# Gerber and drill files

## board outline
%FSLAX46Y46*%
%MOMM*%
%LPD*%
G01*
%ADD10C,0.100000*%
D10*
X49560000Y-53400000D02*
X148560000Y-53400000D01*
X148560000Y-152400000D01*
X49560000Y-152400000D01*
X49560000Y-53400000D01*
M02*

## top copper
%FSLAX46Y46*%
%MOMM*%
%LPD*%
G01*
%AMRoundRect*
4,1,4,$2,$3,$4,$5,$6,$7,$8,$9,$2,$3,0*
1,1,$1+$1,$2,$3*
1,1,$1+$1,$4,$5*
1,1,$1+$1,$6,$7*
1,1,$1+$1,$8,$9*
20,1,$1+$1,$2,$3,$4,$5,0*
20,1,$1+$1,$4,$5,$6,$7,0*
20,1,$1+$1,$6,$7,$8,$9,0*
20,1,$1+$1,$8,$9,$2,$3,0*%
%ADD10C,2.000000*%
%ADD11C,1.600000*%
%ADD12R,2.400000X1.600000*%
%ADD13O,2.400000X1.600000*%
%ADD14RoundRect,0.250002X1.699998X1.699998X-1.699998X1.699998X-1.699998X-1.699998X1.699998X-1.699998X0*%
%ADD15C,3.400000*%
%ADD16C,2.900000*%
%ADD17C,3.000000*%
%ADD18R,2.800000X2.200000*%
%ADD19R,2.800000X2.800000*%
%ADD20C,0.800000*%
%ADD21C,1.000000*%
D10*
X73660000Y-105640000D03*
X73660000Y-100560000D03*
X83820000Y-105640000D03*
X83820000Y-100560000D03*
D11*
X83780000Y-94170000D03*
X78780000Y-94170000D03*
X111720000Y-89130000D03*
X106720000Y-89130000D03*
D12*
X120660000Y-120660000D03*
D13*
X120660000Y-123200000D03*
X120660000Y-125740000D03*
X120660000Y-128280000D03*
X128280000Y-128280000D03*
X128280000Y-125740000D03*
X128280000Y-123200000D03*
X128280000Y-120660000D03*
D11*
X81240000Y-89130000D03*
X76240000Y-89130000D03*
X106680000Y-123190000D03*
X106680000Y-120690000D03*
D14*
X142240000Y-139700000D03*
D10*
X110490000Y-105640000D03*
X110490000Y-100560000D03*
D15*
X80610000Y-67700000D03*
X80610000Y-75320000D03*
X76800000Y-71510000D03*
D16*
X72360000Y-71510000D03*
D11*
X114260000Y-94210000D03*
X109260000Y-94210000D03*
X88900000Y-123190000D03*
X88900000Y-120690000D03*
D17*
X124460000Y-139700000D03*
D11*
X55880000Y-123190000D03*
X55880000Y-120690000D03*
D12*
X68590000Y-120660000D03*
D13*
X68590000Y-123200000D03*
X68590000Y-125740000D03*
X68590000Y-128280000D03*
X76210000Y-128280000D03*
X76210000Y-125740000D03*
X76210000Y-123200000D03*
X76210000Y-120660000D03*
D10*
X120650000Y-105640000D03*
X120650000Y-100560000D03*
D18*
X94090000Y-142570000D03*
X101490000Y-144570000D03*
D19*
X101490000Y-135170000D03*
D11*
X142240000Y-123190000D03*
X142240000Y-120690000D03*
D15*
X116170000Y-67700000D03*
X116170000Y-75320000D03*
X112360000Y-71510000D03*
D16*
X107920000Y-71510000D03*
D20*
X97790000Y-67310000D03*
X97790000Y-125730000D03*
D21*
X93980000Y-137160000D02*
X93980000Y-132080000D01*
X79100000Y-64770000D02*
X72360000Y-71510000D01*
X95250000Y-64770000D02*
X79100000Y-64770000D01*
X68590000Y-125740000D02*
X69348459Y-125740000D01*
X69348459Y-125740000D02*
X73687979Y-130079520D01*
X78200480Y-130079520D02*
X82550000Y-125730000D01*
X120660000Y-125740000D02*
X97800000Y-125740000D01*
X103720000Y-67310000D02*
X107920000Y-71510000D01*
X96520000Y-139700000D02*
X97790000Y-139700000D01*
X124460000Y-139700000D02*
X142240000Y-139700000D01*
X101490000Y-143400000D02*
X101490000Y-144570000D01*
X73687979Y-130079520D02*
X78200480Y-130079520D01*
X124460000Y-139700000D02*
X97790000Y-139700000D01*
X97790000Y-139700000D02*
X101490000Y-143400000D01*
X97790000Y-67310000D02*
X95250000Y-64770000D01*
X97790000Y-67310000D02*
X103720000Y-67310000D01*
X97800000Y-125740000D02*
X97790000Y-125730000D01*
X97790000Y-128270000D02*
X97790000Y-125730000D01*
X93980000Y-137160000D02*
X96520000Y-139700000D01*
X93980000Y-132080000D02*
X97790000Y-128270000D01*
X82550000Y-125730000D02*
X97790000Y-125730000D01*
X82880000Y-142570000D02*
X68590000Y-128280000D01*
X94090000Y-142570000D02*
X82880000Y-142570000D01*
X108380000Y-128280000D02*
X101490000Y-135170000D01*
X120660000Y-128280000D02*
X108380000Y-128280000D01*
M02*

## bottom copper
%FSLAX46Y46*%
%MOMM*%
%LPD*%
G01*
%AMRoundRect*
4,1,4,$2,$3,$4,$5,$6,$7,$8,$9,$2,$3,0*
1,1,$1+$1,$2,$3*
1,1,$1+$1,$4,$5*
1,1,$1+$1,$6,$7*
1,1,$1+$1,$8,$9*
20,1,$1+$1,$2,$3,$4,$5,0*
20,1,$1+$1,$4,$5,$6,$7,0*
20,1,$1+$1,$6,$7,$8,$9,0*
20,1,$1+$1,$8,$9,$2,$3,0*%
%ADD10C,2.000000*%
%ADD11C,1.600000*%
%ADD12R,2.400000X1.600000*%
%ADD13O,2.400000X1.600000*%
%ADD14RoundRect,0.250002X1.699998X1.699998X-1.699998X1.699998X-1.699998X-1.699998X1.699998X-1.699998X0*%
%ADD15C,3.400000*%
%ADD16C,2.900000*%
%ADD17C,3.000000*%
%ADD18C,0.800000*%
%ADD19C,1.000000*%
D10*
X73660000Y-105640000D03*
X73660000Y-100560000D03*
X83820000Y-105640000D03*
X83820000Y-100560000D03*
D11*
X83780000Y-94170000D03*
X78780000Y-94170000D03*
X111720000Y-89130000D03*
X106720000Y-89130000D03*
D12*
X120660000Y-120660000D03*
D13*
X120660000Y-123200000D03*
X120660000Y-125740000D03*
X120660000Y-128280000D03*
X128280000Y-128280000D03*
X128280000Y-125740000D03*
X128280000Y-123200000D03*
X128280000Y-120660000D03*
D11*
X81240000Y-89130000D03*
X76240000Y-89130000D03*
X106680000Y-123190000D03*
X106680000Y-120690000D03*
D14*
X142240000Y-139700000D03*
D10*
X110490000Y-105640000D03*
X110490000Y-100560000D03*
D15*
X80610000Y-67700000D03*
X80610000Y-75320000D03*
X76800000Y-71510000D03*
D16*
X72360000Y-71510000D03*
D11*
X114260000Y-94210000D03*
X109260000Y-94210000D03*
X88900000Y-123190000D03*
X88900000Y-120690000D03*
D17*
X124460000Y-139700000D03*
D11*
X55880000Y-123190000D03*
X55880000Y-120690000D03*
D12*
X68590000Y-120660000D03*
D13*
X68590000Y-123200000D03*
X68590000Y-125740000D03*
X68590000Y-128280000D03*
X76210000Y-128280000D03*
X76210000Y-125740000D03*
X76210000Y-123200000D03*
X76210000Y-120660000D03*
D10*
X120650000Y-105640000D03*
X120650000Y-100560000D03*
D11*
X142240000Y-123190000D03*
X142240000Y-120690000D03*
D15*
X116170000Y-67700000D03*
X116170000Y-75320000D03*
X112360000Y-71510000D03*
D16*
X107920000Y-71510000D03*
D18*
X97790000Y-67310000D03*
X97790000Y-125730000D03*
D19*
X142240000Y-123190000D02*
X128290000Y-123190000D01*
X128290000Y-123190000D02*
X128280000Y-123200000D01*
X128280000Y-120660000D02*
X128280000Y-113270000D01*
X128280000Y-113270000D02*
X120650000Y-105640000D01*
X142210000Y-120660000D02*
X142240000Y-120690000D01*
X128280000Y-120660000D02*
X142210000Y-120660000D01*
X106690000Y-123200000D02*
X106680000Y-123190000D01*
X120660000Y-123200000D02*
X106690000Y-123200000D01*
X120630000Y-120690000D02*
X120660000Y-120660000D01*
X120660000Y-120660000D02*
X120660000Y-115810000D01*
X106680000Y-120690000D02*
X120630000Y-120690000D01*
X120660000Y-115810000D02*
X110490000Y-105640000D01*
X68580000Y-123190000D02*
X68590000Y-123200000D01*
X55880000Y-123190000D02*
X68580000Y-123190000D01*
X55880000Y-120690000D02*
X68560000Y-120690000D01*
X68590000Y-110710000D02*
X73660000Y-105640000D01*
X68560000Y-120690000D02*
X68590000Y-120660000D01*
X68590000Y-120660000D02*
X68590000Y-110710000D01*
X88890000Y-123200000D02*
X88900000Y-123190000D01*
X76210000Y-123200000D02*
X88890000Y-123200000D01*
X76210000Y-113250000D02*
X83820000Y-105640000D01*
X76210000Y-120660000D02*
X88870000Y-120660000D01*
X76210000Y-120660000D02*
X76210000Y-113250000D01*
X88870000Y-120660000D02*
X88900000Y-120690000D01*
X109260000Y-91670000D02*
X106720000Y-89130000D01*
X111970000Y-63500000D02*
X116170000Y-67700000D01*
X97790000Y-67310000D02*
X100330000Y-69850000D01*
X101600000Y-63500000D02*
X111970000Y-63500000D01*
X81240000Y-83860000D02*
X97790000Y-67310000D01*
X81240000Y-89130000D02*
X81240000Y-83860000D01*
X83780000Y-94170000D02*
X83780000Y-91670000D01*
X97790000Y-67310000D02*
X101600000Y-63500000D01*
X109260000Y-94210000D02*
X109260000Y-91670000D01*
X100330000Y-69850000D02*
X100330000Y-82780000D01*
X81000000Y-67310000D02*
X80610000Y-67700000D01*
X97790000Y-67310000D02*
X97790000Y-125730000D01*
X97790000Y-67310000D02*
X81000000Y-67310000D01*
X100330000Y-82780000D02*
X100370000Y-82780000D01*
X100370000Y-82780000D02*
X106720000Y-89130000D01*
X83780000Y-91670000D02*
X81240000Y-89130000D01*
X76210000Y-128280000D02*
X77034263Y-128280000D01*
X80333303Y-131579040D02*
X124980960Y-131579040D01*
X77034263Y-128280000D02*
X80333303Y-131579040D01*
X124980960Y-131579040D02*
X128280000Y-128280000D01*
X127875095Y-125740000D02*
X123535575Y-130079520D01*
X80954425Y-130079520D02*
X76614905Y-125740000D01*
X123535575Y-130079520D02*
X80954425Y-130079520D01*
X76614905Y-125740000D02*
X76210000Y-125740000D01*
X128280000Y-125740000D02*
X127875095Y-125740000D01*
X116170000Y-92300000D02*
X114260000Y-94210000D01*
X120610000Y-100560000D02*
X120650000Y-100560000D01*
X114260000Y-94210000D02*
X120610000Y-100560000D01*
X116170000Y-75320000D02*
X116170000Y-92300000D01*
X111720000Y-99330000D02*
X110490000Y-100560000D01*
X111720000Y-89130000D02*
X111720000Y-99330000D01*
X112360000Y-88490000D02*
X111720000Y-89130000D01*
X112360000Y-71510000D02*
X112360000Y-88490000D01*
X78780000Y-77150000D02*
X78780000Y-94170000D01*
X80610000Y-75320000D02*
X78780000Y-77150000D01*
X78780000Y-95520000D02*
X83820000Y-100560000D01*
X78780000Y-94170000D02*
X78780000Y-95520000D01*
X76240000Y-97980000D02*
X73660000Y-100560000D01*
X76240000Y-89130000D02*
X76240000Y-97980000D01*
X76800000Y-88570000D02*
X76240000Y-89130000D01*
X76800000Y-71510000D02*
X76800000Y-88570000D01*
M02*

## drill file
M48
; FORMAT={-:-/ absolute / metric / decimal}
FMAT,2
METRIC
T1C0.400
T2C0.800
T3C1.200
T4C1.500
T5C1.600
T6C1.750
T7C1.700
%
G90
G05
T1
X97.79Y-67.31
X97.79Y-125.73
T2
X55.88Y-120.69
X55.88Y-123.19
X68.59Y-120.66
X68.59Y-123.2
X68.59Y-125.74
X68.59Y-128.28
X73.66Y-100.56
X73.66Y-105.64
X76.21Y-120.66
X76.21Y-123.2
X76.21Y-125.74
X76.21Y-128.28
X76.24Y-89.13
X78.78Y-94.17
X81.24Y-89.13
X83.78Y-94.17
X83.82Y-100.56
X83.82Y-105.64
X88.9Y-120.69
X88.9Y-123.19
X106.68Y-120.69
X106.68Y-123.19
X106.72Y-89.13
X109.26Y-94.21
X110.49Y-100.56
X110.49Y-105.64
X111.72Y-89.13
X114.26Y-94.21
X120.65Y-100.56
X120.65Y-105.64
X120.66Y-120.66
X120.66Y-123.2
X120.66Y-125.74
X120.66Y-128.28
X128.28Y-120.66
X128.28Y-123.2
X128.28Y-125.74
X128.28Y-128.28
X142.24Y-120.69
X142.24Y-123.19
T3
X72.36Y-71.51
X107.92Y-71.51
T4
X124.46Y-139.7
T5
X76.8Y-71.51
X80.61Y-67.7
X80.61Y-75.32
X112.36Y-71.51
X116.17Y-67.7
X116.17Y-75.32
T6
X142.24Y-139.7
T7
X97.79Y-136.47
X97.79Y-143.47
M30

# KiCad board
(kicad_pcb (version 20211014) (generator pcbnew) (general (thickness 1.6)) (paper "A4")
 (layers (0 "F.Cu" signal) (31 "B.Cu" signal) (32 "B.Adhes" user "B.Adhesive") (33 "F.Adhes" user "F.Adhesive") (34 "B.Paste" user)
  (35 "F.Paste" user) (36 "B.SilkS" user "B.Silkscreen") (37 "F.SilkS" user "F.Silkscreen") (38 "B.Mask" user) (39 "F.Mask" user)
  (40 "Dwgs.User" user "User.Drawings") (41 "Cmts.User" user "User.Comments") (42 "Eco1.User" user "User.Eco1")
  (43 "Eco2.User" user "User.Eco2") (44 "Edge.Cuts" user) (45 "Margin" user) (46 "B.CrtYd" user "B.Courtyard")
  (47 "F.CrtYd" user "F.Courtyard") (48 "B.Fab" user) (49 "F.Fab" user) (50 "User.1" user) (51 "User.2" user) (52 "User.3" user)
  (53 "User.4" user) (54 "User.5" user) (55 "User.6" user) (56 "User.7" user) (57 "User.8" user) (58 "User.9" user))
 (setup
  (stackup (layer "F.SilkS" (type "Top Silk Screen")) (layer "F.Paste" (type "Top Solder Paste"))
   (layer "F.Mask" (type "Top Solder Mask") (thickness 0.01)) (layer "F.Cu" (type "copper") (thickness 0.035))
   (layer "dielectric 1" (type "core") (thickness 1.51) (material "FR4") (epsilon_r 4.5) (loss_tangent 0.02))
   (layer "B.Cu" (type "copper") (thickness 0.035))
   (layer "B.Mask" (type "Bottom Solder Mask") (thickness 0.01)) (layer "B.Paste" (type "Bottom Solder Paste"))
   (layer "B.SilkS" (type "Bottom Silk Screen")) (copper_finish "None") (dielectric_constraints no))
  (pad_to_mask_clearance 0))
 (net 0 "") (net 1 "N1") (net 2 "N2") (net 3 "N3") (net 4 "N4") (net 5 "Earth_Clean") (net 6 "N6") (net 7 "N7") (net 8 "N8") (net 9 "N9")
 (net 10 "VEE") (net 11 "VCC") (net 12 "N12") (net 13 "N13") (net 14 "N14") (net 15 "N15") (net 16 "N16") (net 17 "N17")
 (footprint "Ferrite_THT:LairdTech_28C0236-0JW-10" (layer "F.Cu") (at 73.66 105.64 90)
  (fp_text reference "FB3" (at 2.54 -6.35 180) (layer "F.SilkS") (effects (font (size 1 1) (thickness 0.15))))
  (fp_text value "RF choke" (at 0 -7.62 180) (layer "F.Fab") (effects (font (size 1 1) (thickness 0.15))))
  (pad "1" thru_hole circle (at 0 0 90) (size 2 2) (drill 0.8) (layers *.Cu *.Mask) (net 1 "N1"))
  (pad "2" thru_hole circle (at 5.08 0 90) (size 2 2) (drill 0.8) (layers *.Cu *.Mask) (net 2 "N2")))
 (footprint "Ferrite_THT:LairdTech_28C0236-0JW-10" (layer "F.Cu") (at 83.82 105.64 90)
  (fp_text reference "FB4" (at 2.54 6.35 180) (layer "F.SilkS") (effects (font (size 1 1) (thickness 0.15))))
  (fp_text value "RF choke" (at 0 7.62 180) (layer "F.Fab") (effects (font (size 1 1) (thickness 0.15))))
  (pad "1" thru_hole circle (at 0 0 90) (size 2 2) (drill 0.8) (layers *.Cu *.Mask) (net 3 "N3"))
  (pad "2" thru_hole circle (at 5.08 0 90) (size 2 2) (drill 0.8) (layers *.Cu *.Mask) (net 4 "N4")))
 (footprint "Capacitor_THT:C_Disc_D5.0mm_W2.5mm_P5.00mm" (layer "F.Cu") (at 83.78 94.17 180)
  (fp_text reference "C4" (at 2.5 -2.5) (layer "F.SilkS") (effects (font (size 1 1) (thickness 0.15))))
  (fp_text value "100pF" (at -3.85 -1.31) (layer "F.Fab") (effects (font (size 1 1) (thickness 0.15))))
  (pad "1" thru_hole circle (at 0 0 180) (size 1.6 1.6) (drill 0.8) (layers *.Cu *.Mask) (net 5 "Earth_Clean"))
  (pad "2" thru_hole circle (at 5 0 180) (size 1.6 1.6) (drill 0.8) (layers *.Cu *.Mask) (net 4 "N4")))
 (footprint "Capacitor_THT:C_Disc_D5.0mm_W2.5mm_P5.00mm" (layer "F.Cu") (at 111.72 89.13 180)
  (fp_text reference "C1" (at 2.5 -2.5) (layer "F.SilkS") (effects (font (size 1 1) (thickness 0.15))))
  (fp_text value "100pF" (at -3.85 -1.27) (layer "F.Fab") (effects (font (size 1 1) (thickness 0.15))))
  (pad "1" thru_hole circle (at 0 0 180) (size 1.6 1.6) (drill 0.8) (layers *.Cu *.Mask) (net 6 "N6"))
  (pad "2" thru_hole circle (at 5 0 180) (size 1.6 1.6) (drill 0.8) (layers *.Cu *.Mask) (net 5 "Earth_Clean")))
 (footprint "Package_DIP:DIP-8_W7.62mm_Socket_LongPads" (layer "F.Cu") (at 120.66 120.66)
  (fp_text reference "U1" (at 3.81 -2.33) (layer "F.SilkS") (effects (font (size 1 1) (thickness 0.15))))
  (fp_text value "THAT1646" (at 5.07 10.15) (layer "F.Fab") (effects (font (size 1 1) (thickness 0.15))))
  (pad "1" thru_hole rect (at 0 0) (size 2.4 1.6) (drill 0.8) (layers *.Cu *.Mask) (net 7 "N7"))
  (pad "2" thru_hole oval (at 0 2.54) (size 2.4 1.6) (drill 0.8) (layers *.Cu *.Mask) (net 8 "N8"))
  (pad "3" thru_hole oval (at 0 5.08) (size 2.4 1.6) (drill 0.8) (layers *.Cu *.Mask) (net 5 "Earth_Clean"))
  (pad "4" thru_hole oval (at 0 7.62) (size 2.4 1.6) (drill 0.8) (layers *.Cu *.Mask) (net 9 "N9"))
  (pad "5" thru_hole oval (at 7.62 7.62) (size 2.4 1.6) (drill 0.8) (layers *.Cu *.Mask) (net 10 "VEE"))
  (pad "6" thru_hole oval (at 7.62 5.08) (size 2.4 1.6) (drill 0.8) (layers *.Cu *.Mask) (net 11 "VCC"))
  (pad "7" thru_hole oval (at 7.62 2.54) (size 2.4 1.6) (drill 0.8) (layers *.Cu *.Mask) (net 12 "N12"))
  (pad "8" thru_hole oval (at 7.62 0) (size 2.4 1.6) (drill 0.8) (layers *.Cu *.Mask) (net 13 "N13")))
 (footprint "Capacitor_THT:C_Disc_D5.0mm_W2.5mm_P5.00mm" (layer "F.Cu") (at 81.24 89.13 180)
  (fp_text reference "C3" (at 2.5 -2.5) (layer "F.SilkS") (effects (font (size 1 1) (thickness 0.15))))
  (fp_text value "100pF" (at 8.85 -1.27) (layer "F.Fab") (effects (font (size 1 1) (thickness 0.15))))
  (pad "1" thru_hole circle (at 0 0 180) (size 1.6 1.6) (drill 0.8) (layers *.Cu *.Mask) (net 5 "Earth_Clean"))
  (pad "2" thru_hole circle (at 5 0 180) (size 1.6 1.6) (drill 0.8) (layers *.Cu *.Mask) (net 2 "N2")))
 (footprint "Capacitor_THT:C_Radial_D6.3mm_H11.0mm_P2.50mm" (layer "F.Cu") (at 106.68 123.19 90)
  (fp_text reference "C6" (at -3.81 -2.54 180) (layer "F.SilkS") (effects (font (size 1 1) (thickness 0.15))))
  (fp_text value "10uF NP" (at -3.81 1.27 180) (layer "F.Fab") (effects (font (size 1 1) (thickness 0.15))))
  (pad "1" thru_hole circle (at 0 0 90) (size 1.6 1.6) (drill 0.8) (layers *.Cu *.Mask) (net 8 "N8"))
  (pad "2" thru_hole circle (at 2.5 0 90) (size 1.6 1.6) (drill 0.8) (layers *.Cu *.Mask) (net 7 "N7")))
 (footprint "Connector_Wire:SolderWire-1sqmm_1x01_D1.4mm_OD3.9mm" (layer "F.Cu") (at 142.24 139.7 180)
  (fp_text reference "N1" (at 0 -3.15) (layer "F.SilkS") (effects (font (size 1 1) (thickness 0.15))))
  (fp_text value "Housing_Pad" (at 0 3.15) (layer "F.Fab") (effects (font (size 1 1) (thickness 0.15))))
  (pad "1" thru_hole roundrect (at 0 0 180) (size 3.9 3.9) (drill 1.75) (layers *.Cu *.Mask) (roundrect_rratio 0.06410307692)
   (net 5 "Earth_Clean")))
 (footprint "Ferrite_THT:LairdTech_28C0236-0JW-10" (layer "F.Cu") (at 110.49 105.64 90)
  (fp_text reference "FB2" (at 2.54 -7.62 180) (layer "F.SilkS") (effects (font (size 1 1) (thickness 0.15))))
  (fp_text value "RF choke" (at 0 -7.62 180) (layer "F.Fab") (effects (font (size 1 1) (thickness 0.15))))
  (pad "1" thru_hole circle (at 0 0 90) (size 2 2) (drill 0.8) (layers *.Cu *.Mask) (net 7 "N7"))
  (pad "2" thru_hole circle (at 5.08 0 90) (size 2 2) (drill 0.8) (layers *.Cu *.Mask) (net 6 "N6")))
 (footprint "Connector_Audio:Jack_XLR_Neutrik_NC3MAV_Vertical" (layer "F.Cu") (at 80.61 67.7 -90)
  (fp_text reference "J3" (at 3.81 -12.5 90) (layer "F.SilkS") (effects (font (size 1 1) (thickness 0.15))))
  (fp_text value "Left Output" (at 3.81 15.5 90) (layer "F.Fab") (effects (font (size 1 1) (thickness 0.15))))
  (pad "1" thru_hole circle (at 0 0 270) (size 3.4 3.4) (drill 1.6) (layers *.Cu *.Mask) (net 5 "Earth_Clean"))
  (pad "2" thru_hole circle (at 7.62 0 270) (size 3.4 3.4) (drill 1.6) (layers *.Cu *.Mask) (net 4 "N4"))
  (pad "3" thru_hole circle (at 3.81 3.81 270) (size 3.4 3.4) (drill 1.6) (layers *.Cu *.Mask) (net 2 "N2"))
  (pad "G" thru_hole circle (at 3.81 8.25 270) (size 2.9 2.9) (drill 1.2) (layers *.Cu *.Mask) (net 5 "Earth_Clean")))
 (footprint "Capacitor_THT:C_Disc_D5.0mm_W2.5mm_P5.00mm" (layer "F.Cu") (at 114.26 94.21 180)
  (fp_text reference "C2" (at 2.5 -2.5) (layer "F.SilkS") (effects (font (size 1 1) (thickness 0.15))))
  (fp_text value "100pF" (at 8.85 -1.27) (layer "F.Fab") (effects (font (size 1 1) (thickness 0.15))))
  (pad "1" thru_hole circle (at 0 0 180) (size 1.6 1.6) (drill 0.8) (layers *.Cu *.Mask) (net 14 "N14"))
  (pad "2" thru_hole circle (at 5 0 180) (size 1.6 1.6) (drill 0.8) (layers *.Cu *.Mask) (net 5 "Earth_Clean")))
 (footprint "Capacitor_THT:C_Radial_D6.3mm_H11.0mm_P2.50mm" (layer "F.Cu") (at 88.9 123.19 90)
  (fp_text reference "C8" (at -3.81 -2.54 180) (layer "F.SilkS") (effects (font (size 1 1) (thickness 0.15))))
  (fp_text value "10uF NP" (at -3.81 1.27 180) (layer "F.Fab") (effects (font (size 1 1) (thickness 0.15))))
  (pad "1" thru_hole circle (at 0 0 90) (size 1.6 1.6) (drill 0.8) (layers *.Cu *.Mask) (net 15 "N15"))
  (pad "2" thru_hole circle (at 2.5 0 90) (size 1.6 1.6) (drill 0.8) (layers *.Cu *.Mask) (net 3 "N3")))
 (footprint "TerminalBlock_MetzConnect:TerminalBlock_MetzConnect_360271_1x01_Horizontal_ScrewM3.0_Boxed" (layer "F.Cu")
  (at 124.46 139.7 180)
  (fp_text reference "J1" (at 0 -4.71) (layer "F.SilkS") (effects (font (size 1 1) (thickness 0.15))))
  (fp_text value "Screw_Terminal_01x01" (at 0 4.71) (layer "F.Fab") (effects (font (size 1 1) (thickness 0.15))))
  (pad "1" thru_hole circle (at 0 0 180) (size 3 3) (drill 1.5) (layers *.Cu *.Mask) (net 5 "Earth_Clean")))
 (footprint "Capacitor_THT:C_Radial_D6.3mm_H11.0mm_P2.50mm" (layer "F.Cu") (at 55.88 123.19 90)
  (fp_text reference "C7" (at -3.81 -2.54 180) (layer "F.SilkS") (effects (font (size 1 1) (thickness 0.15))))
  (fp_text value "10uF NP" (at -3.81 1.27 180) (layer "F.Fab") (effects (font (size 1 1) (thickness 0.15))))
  (pad "1" thru_hole circle (at 0 0 90) (size 1.6 1.6) (drill 0.8) (layers *.Cu *.Mask) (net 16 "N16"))
  (pad "2" thru_hole circle (at 2.5 0 90) (size 1.6 1.6) (drill 0.8) (layers *.Cu *.Mask) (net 1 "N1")))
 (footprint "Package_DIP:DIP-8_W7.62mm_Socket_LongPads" (layer "F.Cu") (at 68.59 120.66)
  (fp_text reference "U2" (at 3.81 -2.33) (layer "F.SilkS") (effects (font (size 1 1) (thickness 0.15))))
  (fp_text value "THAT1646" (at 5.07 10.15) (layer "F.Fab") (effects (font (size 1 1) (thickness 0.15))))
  (pad "1" thru_hole rect (at 0 0) (size 2.4 1.6) (drill 0.8) (layers *.Cu *.Mask) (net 1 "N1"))
  (pad "2" thru_hole oval (at 0 2.54) (size 2.4 1.6) (drill 0.8) (layers *.Cu *.Mask) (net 16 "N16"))
  (pad "3" thru_hole oval (at 0 5.08) (size 2.4 1.6) (drill 0.8) (layers *.Cu *.Mask) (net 5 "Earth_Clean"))
  (pad "4" thru_hole oval (at 0 7.62) (size 2.4 1.6) (drill 0.8) (layers *.Cu *.Mask) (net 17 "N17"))
  (pad "5" thru_hole oval (at 7.62 7.62) (size 2.4 1.6) (drill 0.8) (layers *.Cu *.Mask) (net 10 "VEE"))
  (pad "6" thru_hole oval (at 7.62 5.08) (size 2.4 1.6) (drill 0.8) (layers *.Cu *.Mask) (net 11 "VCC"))
  (pad "7" thru_hole oval (at 7.62 2.54) (size 2.4 1.6) (drill 0.8) (layers *.Cu *.Mask) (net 15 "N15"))
  (pad "8" thru_hole oval (at 7.62 0) (size 2.4 1.6) (drill 0.8) (layers *.Cu *.Mask) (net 3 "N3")))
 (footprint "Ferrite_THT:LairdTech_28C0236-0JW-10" (layer "F.Cu") (at 120.65 105.64 90)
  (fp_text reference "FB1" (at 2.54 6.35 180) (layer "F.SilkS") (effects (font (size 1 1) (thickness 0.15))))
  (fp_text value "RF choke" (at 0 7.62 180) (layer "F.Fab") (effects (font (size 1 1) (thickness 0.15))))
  (pad "1" thru_hole circle (at 0 0 90) (size 2 2) (drill 0.8) (layers *.Cu *.Mask) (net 13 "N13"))
  (pad "2" thru_hole circle (at 5.08 0 90) (size 2 2) (drill 0.8) (layers *.Cu *.Mask) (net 14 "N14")))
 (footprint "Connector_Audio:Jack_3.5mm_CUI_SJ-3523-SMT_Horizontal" (layer "F.Cu") (at 97.79 140.97 180)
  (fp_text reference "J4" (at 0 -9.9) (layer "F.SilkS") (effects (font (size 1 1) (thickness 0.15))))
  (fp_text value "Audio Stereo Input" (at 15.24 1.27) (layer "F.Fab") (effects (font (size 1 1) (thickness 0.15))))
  (pad "" np_thru_hole circle (at 0 4.5 180) (size 1.7 1.7) (drill 1.7) (layers *.Cu *.Mask))
  (pad "" np_thru_hole circle (at 0 -2.5 180) (size 1.7 1.7) (drill 1.7) (layers *.Cu *.Mask))
  (pad "R" smd rect (at 3.7 -1.6 180) (size 2.8 2.2) (layers "F.Cu" "F.Paste" "F.Mask") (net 17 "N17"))
  (pad "S" smd rect (at -3.7 -3.6 180) (size 2.8 2.2) (layers "F.Cu" "F.Paste" "F.Mask") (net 5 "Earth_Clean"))
  (pad "T" smd rect (at -3.7 5.8 180) (size 2.8 2.8) (layers "F.Cu" "F.Paste" "F.Mask") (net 9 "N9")))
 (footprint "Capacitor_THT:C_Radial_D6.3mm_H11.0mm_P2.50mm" (layer "F.Cu") (at 142.24 123.19 90)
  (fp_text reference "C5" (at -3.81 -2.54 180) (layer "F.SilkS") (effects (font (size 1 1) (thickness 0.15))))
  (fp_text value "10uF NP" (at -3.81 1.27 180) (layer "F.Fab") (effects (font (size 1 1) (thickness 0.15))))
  (pad "1" thru_hole circle (at 0 0 90) (size 1.6 1.6) (drill 0.8) (layers *.Cu *.Mask) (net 12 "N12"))
  (pad "2" thru_hole circle (at 2.5 0 90) (size 1.6 1.6) (drill 0.8) (layers *.Cu *.Mask) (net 13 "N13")))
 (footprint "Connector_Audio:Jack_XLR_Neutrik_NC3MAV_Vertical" (layer "F.Cu") (at 116.17 67.7 -90)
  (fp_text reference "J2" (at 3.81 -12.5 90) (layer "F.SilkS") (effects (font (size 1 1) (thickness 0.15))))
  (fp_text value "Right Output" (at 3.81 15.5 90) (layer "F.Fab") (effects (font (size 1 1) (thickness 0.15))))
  (pad "1" thru_hole circle (at 0 0 270) (size 3.4 3.4) (drill 1.6) (layers *.Cu *.Mask) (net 5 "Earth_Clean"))
  (pad "2" thru_hole circle (at 7.62 0 270) (size 3.4 3.4) (drill 1.6) (layers *.Cu *.Mask) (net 14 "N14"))
  (pad "3" thru_hole circle (at 3.81 3.81 270) (size 3.4 3.4) (drill 1.6) (layers *.Cu *.Mask) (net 6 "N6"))
  (pad "G" thru_hole circle (at 3.81 8.25 270) (size 2.9 2.9) (drill 1.2) (layers *.Cu *.Mask) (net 5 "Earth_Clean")))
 (gr_rect (start 148.56 53.4) (end 49.56 152.4) (layer "Edge.Cuts") (width 0.1) (fill none))
 (segment (start 142.24 123.19) (end 128.29 123.19) (width 1) (layer "B.Cu") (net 12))
 (segment (start 128.29 123.19) (end 128.28 123.2) (width 1) (layer "B.Cu") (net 12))
 (segment (start 128.28 120.66) (end 128.28 113.27) (width 1) (layer "B.Cu") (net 13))
 (segment (start 128.28 113.27) (end 120.65 105.64) (width 1) (layer "B.Cu") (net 13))
 (segment (start 142.21 120.66) (end 142.24 120.69) (width 1) (layer "B.Cu") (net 13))
 (segment (start 128.28 120.66) (end 142.21 120.66) (width 1) (layer "B.Cu") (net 13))
 (segment (start 106.69 123.2) (end 106.68 123.19) (width 1) (layer "B.Cu") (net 8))
 (segment (start 120.66 123.2) (end 106.69 123.2) (width 1) (layer "B.Cu") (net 8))
 (segment (start 120.63 120.69) (end 120.66 120.66) (width 1) (layer "B.Cu") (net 7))
 (segment (start 120.66 120.66) (end 120.66 115.81) (width 1) (layer "B.Cu") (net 7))
 (segment (start 106.68 120.69) (end 120.63 120.69) (width 1) (layer "B.Cu") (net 7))
 (segment (start 120.66 115.81) (end 110.49 105.64) (width 1) (layer "B.Cu") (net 7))
 (segment (start 68.58 123.19) (end 68.59 123.2) (width 1) (layer "B.Cu") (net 16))
 (segment (start 55.88 123.19) (end 68.58 123.19) (width 1) (layer "B.Cu") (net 16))
 (segment (start 55.88 120.69) (end 68.56 120.69) (width 1) (layer "B.Cu") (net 1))
 (segment (start 68.59 110.71) (end 73.66 105.64) (width 1) (layer "B.Cu") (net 1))
 (segment (start 68.56 120.69) (end 68.59 120.66) (width 1) (layer "B.Cu") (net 1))
 (segment (start 68.59 120.66) (end 68.59 110.71) (width 1) (layer "B.Cu") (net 1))
 (segment (start 88.89 123.2) (end 88.9 123.19) (width 1) (layer "B.Cu") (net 15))
 (segment (start 76.21 123.2) (end 88.89 123.2) (width 1) (layer "B.Cu") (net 15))
 (segment (start 76.21 113.25) (end 83.82 105.64) (width 1) (layer "B.Cu") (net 3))
 (segment (start 76.21 120.66) (end 88.87 120.66) (width 1) (layer "B.Cu") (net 3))
 (segment (start 76.21 120.66) (end 76.21 113.25) (width 1) (layer "B.Cu") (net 3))
 (segment (start 88.87 120.66) (end 88.9 120.69) (width 1) (layer "B.Cu") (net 3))
 (segment (start 93.98 137.16) (end 93.98 132.08) (width 1) (layer "F.Cu") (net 5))
 (segment (start 79.1 64.77) (end 72.36 71.51) (width 1) (layer "F.Cu") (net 5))
 (segment (start 95.25 64.77) (end 79.1 64.77) (width 1) (layer "F.Cu") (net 5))
 (segment (start 68.59 125.74) (end 69.348459 125.74) (width 1) (layer "F.Cu") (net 5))
 (segment (start 69.348459 125.74) (end 73.687979 130.07952) (width 1) (layer "F.Cu") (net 5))
 (segment (start 78.20048 130.07952) (end 82.55 125.73) (width 1) (layer "F.Cu") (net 5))
 (segment (start 120.66 125.74) (end 97.8 125.74) (width 1) (layer "F.Cu") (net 5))
 (segment (start 103.72 67.31) (end 107.92 71.51) (width 1) (layer "F.Cu") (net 5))
 (segment (start 96.52 139.7) (end 97.79 139.7) (width 1) (layer "F.Cu") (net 5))
 (segment (start 124.46 139.7) (end 142.24 139.7) (width 1) (layer "F.Cu") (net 5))
 (segment (start 101.49 143.4) (end 101.49 144.57) (width 1) (layer "F.Cu") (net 5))
 (segment (start 73.687979 130.07952) (end 78.20048 130.07952) (width 1) (layer "F.Cu") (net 5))
 (segment (start 124.46 139.7) (end 97.79 139.7) (width 1) (layer "F.Cu") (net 5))
 (segment (start 97.79 139.7) (end 101.49 143.4) (width 1) (layer "F.Cu") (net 5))
 (segment (start 97.79 67.31) (end 95.25 64.77) (width 1) (layer "F.Cu") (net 5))
 (segment (start 97.79 67.31) (end 103.72 67.31) (width 1) (layer "F.Cu") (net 5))
 (segment (start 97.8 125.74) (end 97.79 125.73) (width 1) (layer "F.Cu") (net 5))
 (segment (start 97.79 128.27) (end 97.79 125.73) (width 1) (layer "F.Cu") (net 5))
 (segment (start 93.98 137.16) (end 96.52 139.7) (width 1) (layer "F.Cu") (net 5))
 (segment (start 93.98 132.08) (end 97.79 128.27) (width 1) (layer "F.Cu") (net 5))
 (segment (start 82.55 125.73) (end 97.79 125.73) (width 1) (layer "F.Cu") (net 5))
 (via (at 97.79 67.31) (size 0.8) (drill 0.4) (layers "F.Cu" "B.Cu") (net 5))
 (via (at 97.79 125.73) (size 0.8) (drill 0.4) (layers "F.Cu" "B.Cu") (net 5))
 (segment (start 109.26 91.67) (end 106.72 89.13) (width 1) (layer "B.Cu") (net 5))
 (segment (start 111.97 63.5) (end 116.17 67.7) (width 1) (layer "B.Cu") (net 5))
 (segment (start 97.79 67.31) (end 100.33 69.85) (width 1) (layer "B.Cu") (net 5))
 (segment (start 101.6 63.5) (end 111.97 63.5) (width 1) (layer "B.Cu") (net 5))
 (segment (start 81.24 83.86) (end 97.79 67.31) (width 1) (layer "B.Cu") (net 5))
 (segment (start 81.24 89.13) (end 81.24 83.86) (width 1) (layer "B.Cu") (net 5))
 (segment (start 83.78 94.17) (end 83.78 91.67) (width 1) (layer "B.Cu") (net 5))
 (segment (start 97.79 67.31) (end 101.6 63.5) (width 1) (layer "B.Cu") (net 5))
 (segment (start 109.26 94.21) (end 109.26 91.67) (width 1) (layer "B.Cu") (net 5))
 (segment (start 100.33 69.85) (end 100.33 82.78) (width 1) (layer "B.Cu") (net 5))
 (segment (start 81 67.31) (end 80.61 67.7) (width 1) (layer "B.Cu") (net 5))
 (segment (start 97.79 67.31) (end 97.79 125.73) (width 1) (layer "B.Cu") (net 5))
 (segment (start 97.79 67.31) (end 81 67.31) (width 1) (layer "B.Cu") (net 5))
 (segment (start 100.33 82.78) (end 100.37 82.78) (width 1) (layer "B.Cu") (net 5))
 (segment (start 100.37 82.78) (end 106.72 89.13) (width 1) (layer "B.Cu") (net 5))
 (segment (start 83.78 91.67) (end 81.24 89.13) (width 1) (layer "B.Cu") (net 5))
 (segment (start 82.88 142.57) (end 68.59 128.28) (width 1) (layer "F.Cu") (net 17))
 (segment (start 94.09 142.57) (end 82.88 142.57) (width 1) (layer "F.Cu") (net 17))
 (segment (start 76.21 128.28) (end 77.034263 128.28) (width 1) (layer "B.Cu") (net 10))
 (segment (start 80.333303 131.57904) (end 124.98096 131.57904) (width 1) (layer "B.Cu") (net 10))
 (segment (start 77.034263 128.28) (end 80.333303 131.57904) (width 1) (layer "B.Cu") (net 10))
 (segment (start 124.98096 131.57904) (end 128.28 128.28) (width 1) (layer "B.Cu") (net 10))
 (segment (start 127.875095 125.74) (end 123.535575 130.07952) (width 1) (layer "B.Cu") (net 11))
 (segment (start 80.954425 130.07952) (end 76.614905 125.74) (width 1) (layer "B.Cu") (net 11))
 (segment (start 123.535575 130.07952) (end 80.954425 130.07952) (width 1) (layer "B.Cu") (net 11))
 (segment (start 76.614905 125.74) (end 76.21 125.74) (width 1) (layer "B.Cu") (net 11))
 (segment (start 128.28 125.74) (end 127.875095 125.74) (width 1) (layer "B.Cu") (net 11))
 (segment (start 108.38 128.28) (end 101.49 135.17) (width 1) (layer "F.Cu") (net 9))
 (segment (start 120.66 128.28) (end 108.38 128.28) (width 1) (layer "F.Cu") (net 9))
 (segment (start 116.17 92.3) (end 114.26 94.21) (width 1) (layer "B.Cu") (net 14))
 (segment (start 120.61 100.56) (end 120.65 100.56) (width 1) (layer "B.Cu") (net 14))
 (segment (start 114.26 94.21) (end 120.61 100.56) (width 1) (layer "B.Cu") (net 14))
 (segment (start 116.17 75.32) (end 116.17 92.3) (width 1) (layer "B.Cu") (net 14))
 (segment (start 111.72 99.33) (end 110.49 100.56) (width 1) (layer "B.Cu") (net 6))
 (segment (start 111.72 89.13) (end 111.72 99.33) (width 1) (layer "B.Cu") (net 6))
 (segment (start 112.36 88.49) (end 111.72 89.13) (width 1) (layer "B.Cu") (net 6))
 (segment (start 112.36 71.51) (end 112.36 88.49) (width 1) (layer "B.Cu") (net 6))
 (segment (start 78.78 77.15) (end 78.78 94.17) (width 1) (layer "B.Cu") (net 4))
 (segment (start 80.61 75.32) (end 78.78 77.15) (width 1) (layer "B.Cu") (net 4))
 (segment (start 78.78 95.52) (end 83.82 100.56) (width 1) (layer "B.Cu") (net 4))
 (segment (start 78.78 94.17) (end 78.78 95.52) (width 1) (layer "B.Cu") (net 4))
 (segment (start 76.24 97.98) (end 73.66 100.56) (width 1) (layer "B.Cu") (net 2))
 (segment (start 76.24 89.13) (end 76.24 97.98) (width 1) (layer "B.Cu") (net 2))
 (segment (start 76.8 88.57) (end 76.24 89.13) (width 1) (layer "B.Cu") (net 2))
 (segment (start 76.8 71.51) (end 76.8 88.57) (width 1) (layer "B.Cu") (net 2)))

